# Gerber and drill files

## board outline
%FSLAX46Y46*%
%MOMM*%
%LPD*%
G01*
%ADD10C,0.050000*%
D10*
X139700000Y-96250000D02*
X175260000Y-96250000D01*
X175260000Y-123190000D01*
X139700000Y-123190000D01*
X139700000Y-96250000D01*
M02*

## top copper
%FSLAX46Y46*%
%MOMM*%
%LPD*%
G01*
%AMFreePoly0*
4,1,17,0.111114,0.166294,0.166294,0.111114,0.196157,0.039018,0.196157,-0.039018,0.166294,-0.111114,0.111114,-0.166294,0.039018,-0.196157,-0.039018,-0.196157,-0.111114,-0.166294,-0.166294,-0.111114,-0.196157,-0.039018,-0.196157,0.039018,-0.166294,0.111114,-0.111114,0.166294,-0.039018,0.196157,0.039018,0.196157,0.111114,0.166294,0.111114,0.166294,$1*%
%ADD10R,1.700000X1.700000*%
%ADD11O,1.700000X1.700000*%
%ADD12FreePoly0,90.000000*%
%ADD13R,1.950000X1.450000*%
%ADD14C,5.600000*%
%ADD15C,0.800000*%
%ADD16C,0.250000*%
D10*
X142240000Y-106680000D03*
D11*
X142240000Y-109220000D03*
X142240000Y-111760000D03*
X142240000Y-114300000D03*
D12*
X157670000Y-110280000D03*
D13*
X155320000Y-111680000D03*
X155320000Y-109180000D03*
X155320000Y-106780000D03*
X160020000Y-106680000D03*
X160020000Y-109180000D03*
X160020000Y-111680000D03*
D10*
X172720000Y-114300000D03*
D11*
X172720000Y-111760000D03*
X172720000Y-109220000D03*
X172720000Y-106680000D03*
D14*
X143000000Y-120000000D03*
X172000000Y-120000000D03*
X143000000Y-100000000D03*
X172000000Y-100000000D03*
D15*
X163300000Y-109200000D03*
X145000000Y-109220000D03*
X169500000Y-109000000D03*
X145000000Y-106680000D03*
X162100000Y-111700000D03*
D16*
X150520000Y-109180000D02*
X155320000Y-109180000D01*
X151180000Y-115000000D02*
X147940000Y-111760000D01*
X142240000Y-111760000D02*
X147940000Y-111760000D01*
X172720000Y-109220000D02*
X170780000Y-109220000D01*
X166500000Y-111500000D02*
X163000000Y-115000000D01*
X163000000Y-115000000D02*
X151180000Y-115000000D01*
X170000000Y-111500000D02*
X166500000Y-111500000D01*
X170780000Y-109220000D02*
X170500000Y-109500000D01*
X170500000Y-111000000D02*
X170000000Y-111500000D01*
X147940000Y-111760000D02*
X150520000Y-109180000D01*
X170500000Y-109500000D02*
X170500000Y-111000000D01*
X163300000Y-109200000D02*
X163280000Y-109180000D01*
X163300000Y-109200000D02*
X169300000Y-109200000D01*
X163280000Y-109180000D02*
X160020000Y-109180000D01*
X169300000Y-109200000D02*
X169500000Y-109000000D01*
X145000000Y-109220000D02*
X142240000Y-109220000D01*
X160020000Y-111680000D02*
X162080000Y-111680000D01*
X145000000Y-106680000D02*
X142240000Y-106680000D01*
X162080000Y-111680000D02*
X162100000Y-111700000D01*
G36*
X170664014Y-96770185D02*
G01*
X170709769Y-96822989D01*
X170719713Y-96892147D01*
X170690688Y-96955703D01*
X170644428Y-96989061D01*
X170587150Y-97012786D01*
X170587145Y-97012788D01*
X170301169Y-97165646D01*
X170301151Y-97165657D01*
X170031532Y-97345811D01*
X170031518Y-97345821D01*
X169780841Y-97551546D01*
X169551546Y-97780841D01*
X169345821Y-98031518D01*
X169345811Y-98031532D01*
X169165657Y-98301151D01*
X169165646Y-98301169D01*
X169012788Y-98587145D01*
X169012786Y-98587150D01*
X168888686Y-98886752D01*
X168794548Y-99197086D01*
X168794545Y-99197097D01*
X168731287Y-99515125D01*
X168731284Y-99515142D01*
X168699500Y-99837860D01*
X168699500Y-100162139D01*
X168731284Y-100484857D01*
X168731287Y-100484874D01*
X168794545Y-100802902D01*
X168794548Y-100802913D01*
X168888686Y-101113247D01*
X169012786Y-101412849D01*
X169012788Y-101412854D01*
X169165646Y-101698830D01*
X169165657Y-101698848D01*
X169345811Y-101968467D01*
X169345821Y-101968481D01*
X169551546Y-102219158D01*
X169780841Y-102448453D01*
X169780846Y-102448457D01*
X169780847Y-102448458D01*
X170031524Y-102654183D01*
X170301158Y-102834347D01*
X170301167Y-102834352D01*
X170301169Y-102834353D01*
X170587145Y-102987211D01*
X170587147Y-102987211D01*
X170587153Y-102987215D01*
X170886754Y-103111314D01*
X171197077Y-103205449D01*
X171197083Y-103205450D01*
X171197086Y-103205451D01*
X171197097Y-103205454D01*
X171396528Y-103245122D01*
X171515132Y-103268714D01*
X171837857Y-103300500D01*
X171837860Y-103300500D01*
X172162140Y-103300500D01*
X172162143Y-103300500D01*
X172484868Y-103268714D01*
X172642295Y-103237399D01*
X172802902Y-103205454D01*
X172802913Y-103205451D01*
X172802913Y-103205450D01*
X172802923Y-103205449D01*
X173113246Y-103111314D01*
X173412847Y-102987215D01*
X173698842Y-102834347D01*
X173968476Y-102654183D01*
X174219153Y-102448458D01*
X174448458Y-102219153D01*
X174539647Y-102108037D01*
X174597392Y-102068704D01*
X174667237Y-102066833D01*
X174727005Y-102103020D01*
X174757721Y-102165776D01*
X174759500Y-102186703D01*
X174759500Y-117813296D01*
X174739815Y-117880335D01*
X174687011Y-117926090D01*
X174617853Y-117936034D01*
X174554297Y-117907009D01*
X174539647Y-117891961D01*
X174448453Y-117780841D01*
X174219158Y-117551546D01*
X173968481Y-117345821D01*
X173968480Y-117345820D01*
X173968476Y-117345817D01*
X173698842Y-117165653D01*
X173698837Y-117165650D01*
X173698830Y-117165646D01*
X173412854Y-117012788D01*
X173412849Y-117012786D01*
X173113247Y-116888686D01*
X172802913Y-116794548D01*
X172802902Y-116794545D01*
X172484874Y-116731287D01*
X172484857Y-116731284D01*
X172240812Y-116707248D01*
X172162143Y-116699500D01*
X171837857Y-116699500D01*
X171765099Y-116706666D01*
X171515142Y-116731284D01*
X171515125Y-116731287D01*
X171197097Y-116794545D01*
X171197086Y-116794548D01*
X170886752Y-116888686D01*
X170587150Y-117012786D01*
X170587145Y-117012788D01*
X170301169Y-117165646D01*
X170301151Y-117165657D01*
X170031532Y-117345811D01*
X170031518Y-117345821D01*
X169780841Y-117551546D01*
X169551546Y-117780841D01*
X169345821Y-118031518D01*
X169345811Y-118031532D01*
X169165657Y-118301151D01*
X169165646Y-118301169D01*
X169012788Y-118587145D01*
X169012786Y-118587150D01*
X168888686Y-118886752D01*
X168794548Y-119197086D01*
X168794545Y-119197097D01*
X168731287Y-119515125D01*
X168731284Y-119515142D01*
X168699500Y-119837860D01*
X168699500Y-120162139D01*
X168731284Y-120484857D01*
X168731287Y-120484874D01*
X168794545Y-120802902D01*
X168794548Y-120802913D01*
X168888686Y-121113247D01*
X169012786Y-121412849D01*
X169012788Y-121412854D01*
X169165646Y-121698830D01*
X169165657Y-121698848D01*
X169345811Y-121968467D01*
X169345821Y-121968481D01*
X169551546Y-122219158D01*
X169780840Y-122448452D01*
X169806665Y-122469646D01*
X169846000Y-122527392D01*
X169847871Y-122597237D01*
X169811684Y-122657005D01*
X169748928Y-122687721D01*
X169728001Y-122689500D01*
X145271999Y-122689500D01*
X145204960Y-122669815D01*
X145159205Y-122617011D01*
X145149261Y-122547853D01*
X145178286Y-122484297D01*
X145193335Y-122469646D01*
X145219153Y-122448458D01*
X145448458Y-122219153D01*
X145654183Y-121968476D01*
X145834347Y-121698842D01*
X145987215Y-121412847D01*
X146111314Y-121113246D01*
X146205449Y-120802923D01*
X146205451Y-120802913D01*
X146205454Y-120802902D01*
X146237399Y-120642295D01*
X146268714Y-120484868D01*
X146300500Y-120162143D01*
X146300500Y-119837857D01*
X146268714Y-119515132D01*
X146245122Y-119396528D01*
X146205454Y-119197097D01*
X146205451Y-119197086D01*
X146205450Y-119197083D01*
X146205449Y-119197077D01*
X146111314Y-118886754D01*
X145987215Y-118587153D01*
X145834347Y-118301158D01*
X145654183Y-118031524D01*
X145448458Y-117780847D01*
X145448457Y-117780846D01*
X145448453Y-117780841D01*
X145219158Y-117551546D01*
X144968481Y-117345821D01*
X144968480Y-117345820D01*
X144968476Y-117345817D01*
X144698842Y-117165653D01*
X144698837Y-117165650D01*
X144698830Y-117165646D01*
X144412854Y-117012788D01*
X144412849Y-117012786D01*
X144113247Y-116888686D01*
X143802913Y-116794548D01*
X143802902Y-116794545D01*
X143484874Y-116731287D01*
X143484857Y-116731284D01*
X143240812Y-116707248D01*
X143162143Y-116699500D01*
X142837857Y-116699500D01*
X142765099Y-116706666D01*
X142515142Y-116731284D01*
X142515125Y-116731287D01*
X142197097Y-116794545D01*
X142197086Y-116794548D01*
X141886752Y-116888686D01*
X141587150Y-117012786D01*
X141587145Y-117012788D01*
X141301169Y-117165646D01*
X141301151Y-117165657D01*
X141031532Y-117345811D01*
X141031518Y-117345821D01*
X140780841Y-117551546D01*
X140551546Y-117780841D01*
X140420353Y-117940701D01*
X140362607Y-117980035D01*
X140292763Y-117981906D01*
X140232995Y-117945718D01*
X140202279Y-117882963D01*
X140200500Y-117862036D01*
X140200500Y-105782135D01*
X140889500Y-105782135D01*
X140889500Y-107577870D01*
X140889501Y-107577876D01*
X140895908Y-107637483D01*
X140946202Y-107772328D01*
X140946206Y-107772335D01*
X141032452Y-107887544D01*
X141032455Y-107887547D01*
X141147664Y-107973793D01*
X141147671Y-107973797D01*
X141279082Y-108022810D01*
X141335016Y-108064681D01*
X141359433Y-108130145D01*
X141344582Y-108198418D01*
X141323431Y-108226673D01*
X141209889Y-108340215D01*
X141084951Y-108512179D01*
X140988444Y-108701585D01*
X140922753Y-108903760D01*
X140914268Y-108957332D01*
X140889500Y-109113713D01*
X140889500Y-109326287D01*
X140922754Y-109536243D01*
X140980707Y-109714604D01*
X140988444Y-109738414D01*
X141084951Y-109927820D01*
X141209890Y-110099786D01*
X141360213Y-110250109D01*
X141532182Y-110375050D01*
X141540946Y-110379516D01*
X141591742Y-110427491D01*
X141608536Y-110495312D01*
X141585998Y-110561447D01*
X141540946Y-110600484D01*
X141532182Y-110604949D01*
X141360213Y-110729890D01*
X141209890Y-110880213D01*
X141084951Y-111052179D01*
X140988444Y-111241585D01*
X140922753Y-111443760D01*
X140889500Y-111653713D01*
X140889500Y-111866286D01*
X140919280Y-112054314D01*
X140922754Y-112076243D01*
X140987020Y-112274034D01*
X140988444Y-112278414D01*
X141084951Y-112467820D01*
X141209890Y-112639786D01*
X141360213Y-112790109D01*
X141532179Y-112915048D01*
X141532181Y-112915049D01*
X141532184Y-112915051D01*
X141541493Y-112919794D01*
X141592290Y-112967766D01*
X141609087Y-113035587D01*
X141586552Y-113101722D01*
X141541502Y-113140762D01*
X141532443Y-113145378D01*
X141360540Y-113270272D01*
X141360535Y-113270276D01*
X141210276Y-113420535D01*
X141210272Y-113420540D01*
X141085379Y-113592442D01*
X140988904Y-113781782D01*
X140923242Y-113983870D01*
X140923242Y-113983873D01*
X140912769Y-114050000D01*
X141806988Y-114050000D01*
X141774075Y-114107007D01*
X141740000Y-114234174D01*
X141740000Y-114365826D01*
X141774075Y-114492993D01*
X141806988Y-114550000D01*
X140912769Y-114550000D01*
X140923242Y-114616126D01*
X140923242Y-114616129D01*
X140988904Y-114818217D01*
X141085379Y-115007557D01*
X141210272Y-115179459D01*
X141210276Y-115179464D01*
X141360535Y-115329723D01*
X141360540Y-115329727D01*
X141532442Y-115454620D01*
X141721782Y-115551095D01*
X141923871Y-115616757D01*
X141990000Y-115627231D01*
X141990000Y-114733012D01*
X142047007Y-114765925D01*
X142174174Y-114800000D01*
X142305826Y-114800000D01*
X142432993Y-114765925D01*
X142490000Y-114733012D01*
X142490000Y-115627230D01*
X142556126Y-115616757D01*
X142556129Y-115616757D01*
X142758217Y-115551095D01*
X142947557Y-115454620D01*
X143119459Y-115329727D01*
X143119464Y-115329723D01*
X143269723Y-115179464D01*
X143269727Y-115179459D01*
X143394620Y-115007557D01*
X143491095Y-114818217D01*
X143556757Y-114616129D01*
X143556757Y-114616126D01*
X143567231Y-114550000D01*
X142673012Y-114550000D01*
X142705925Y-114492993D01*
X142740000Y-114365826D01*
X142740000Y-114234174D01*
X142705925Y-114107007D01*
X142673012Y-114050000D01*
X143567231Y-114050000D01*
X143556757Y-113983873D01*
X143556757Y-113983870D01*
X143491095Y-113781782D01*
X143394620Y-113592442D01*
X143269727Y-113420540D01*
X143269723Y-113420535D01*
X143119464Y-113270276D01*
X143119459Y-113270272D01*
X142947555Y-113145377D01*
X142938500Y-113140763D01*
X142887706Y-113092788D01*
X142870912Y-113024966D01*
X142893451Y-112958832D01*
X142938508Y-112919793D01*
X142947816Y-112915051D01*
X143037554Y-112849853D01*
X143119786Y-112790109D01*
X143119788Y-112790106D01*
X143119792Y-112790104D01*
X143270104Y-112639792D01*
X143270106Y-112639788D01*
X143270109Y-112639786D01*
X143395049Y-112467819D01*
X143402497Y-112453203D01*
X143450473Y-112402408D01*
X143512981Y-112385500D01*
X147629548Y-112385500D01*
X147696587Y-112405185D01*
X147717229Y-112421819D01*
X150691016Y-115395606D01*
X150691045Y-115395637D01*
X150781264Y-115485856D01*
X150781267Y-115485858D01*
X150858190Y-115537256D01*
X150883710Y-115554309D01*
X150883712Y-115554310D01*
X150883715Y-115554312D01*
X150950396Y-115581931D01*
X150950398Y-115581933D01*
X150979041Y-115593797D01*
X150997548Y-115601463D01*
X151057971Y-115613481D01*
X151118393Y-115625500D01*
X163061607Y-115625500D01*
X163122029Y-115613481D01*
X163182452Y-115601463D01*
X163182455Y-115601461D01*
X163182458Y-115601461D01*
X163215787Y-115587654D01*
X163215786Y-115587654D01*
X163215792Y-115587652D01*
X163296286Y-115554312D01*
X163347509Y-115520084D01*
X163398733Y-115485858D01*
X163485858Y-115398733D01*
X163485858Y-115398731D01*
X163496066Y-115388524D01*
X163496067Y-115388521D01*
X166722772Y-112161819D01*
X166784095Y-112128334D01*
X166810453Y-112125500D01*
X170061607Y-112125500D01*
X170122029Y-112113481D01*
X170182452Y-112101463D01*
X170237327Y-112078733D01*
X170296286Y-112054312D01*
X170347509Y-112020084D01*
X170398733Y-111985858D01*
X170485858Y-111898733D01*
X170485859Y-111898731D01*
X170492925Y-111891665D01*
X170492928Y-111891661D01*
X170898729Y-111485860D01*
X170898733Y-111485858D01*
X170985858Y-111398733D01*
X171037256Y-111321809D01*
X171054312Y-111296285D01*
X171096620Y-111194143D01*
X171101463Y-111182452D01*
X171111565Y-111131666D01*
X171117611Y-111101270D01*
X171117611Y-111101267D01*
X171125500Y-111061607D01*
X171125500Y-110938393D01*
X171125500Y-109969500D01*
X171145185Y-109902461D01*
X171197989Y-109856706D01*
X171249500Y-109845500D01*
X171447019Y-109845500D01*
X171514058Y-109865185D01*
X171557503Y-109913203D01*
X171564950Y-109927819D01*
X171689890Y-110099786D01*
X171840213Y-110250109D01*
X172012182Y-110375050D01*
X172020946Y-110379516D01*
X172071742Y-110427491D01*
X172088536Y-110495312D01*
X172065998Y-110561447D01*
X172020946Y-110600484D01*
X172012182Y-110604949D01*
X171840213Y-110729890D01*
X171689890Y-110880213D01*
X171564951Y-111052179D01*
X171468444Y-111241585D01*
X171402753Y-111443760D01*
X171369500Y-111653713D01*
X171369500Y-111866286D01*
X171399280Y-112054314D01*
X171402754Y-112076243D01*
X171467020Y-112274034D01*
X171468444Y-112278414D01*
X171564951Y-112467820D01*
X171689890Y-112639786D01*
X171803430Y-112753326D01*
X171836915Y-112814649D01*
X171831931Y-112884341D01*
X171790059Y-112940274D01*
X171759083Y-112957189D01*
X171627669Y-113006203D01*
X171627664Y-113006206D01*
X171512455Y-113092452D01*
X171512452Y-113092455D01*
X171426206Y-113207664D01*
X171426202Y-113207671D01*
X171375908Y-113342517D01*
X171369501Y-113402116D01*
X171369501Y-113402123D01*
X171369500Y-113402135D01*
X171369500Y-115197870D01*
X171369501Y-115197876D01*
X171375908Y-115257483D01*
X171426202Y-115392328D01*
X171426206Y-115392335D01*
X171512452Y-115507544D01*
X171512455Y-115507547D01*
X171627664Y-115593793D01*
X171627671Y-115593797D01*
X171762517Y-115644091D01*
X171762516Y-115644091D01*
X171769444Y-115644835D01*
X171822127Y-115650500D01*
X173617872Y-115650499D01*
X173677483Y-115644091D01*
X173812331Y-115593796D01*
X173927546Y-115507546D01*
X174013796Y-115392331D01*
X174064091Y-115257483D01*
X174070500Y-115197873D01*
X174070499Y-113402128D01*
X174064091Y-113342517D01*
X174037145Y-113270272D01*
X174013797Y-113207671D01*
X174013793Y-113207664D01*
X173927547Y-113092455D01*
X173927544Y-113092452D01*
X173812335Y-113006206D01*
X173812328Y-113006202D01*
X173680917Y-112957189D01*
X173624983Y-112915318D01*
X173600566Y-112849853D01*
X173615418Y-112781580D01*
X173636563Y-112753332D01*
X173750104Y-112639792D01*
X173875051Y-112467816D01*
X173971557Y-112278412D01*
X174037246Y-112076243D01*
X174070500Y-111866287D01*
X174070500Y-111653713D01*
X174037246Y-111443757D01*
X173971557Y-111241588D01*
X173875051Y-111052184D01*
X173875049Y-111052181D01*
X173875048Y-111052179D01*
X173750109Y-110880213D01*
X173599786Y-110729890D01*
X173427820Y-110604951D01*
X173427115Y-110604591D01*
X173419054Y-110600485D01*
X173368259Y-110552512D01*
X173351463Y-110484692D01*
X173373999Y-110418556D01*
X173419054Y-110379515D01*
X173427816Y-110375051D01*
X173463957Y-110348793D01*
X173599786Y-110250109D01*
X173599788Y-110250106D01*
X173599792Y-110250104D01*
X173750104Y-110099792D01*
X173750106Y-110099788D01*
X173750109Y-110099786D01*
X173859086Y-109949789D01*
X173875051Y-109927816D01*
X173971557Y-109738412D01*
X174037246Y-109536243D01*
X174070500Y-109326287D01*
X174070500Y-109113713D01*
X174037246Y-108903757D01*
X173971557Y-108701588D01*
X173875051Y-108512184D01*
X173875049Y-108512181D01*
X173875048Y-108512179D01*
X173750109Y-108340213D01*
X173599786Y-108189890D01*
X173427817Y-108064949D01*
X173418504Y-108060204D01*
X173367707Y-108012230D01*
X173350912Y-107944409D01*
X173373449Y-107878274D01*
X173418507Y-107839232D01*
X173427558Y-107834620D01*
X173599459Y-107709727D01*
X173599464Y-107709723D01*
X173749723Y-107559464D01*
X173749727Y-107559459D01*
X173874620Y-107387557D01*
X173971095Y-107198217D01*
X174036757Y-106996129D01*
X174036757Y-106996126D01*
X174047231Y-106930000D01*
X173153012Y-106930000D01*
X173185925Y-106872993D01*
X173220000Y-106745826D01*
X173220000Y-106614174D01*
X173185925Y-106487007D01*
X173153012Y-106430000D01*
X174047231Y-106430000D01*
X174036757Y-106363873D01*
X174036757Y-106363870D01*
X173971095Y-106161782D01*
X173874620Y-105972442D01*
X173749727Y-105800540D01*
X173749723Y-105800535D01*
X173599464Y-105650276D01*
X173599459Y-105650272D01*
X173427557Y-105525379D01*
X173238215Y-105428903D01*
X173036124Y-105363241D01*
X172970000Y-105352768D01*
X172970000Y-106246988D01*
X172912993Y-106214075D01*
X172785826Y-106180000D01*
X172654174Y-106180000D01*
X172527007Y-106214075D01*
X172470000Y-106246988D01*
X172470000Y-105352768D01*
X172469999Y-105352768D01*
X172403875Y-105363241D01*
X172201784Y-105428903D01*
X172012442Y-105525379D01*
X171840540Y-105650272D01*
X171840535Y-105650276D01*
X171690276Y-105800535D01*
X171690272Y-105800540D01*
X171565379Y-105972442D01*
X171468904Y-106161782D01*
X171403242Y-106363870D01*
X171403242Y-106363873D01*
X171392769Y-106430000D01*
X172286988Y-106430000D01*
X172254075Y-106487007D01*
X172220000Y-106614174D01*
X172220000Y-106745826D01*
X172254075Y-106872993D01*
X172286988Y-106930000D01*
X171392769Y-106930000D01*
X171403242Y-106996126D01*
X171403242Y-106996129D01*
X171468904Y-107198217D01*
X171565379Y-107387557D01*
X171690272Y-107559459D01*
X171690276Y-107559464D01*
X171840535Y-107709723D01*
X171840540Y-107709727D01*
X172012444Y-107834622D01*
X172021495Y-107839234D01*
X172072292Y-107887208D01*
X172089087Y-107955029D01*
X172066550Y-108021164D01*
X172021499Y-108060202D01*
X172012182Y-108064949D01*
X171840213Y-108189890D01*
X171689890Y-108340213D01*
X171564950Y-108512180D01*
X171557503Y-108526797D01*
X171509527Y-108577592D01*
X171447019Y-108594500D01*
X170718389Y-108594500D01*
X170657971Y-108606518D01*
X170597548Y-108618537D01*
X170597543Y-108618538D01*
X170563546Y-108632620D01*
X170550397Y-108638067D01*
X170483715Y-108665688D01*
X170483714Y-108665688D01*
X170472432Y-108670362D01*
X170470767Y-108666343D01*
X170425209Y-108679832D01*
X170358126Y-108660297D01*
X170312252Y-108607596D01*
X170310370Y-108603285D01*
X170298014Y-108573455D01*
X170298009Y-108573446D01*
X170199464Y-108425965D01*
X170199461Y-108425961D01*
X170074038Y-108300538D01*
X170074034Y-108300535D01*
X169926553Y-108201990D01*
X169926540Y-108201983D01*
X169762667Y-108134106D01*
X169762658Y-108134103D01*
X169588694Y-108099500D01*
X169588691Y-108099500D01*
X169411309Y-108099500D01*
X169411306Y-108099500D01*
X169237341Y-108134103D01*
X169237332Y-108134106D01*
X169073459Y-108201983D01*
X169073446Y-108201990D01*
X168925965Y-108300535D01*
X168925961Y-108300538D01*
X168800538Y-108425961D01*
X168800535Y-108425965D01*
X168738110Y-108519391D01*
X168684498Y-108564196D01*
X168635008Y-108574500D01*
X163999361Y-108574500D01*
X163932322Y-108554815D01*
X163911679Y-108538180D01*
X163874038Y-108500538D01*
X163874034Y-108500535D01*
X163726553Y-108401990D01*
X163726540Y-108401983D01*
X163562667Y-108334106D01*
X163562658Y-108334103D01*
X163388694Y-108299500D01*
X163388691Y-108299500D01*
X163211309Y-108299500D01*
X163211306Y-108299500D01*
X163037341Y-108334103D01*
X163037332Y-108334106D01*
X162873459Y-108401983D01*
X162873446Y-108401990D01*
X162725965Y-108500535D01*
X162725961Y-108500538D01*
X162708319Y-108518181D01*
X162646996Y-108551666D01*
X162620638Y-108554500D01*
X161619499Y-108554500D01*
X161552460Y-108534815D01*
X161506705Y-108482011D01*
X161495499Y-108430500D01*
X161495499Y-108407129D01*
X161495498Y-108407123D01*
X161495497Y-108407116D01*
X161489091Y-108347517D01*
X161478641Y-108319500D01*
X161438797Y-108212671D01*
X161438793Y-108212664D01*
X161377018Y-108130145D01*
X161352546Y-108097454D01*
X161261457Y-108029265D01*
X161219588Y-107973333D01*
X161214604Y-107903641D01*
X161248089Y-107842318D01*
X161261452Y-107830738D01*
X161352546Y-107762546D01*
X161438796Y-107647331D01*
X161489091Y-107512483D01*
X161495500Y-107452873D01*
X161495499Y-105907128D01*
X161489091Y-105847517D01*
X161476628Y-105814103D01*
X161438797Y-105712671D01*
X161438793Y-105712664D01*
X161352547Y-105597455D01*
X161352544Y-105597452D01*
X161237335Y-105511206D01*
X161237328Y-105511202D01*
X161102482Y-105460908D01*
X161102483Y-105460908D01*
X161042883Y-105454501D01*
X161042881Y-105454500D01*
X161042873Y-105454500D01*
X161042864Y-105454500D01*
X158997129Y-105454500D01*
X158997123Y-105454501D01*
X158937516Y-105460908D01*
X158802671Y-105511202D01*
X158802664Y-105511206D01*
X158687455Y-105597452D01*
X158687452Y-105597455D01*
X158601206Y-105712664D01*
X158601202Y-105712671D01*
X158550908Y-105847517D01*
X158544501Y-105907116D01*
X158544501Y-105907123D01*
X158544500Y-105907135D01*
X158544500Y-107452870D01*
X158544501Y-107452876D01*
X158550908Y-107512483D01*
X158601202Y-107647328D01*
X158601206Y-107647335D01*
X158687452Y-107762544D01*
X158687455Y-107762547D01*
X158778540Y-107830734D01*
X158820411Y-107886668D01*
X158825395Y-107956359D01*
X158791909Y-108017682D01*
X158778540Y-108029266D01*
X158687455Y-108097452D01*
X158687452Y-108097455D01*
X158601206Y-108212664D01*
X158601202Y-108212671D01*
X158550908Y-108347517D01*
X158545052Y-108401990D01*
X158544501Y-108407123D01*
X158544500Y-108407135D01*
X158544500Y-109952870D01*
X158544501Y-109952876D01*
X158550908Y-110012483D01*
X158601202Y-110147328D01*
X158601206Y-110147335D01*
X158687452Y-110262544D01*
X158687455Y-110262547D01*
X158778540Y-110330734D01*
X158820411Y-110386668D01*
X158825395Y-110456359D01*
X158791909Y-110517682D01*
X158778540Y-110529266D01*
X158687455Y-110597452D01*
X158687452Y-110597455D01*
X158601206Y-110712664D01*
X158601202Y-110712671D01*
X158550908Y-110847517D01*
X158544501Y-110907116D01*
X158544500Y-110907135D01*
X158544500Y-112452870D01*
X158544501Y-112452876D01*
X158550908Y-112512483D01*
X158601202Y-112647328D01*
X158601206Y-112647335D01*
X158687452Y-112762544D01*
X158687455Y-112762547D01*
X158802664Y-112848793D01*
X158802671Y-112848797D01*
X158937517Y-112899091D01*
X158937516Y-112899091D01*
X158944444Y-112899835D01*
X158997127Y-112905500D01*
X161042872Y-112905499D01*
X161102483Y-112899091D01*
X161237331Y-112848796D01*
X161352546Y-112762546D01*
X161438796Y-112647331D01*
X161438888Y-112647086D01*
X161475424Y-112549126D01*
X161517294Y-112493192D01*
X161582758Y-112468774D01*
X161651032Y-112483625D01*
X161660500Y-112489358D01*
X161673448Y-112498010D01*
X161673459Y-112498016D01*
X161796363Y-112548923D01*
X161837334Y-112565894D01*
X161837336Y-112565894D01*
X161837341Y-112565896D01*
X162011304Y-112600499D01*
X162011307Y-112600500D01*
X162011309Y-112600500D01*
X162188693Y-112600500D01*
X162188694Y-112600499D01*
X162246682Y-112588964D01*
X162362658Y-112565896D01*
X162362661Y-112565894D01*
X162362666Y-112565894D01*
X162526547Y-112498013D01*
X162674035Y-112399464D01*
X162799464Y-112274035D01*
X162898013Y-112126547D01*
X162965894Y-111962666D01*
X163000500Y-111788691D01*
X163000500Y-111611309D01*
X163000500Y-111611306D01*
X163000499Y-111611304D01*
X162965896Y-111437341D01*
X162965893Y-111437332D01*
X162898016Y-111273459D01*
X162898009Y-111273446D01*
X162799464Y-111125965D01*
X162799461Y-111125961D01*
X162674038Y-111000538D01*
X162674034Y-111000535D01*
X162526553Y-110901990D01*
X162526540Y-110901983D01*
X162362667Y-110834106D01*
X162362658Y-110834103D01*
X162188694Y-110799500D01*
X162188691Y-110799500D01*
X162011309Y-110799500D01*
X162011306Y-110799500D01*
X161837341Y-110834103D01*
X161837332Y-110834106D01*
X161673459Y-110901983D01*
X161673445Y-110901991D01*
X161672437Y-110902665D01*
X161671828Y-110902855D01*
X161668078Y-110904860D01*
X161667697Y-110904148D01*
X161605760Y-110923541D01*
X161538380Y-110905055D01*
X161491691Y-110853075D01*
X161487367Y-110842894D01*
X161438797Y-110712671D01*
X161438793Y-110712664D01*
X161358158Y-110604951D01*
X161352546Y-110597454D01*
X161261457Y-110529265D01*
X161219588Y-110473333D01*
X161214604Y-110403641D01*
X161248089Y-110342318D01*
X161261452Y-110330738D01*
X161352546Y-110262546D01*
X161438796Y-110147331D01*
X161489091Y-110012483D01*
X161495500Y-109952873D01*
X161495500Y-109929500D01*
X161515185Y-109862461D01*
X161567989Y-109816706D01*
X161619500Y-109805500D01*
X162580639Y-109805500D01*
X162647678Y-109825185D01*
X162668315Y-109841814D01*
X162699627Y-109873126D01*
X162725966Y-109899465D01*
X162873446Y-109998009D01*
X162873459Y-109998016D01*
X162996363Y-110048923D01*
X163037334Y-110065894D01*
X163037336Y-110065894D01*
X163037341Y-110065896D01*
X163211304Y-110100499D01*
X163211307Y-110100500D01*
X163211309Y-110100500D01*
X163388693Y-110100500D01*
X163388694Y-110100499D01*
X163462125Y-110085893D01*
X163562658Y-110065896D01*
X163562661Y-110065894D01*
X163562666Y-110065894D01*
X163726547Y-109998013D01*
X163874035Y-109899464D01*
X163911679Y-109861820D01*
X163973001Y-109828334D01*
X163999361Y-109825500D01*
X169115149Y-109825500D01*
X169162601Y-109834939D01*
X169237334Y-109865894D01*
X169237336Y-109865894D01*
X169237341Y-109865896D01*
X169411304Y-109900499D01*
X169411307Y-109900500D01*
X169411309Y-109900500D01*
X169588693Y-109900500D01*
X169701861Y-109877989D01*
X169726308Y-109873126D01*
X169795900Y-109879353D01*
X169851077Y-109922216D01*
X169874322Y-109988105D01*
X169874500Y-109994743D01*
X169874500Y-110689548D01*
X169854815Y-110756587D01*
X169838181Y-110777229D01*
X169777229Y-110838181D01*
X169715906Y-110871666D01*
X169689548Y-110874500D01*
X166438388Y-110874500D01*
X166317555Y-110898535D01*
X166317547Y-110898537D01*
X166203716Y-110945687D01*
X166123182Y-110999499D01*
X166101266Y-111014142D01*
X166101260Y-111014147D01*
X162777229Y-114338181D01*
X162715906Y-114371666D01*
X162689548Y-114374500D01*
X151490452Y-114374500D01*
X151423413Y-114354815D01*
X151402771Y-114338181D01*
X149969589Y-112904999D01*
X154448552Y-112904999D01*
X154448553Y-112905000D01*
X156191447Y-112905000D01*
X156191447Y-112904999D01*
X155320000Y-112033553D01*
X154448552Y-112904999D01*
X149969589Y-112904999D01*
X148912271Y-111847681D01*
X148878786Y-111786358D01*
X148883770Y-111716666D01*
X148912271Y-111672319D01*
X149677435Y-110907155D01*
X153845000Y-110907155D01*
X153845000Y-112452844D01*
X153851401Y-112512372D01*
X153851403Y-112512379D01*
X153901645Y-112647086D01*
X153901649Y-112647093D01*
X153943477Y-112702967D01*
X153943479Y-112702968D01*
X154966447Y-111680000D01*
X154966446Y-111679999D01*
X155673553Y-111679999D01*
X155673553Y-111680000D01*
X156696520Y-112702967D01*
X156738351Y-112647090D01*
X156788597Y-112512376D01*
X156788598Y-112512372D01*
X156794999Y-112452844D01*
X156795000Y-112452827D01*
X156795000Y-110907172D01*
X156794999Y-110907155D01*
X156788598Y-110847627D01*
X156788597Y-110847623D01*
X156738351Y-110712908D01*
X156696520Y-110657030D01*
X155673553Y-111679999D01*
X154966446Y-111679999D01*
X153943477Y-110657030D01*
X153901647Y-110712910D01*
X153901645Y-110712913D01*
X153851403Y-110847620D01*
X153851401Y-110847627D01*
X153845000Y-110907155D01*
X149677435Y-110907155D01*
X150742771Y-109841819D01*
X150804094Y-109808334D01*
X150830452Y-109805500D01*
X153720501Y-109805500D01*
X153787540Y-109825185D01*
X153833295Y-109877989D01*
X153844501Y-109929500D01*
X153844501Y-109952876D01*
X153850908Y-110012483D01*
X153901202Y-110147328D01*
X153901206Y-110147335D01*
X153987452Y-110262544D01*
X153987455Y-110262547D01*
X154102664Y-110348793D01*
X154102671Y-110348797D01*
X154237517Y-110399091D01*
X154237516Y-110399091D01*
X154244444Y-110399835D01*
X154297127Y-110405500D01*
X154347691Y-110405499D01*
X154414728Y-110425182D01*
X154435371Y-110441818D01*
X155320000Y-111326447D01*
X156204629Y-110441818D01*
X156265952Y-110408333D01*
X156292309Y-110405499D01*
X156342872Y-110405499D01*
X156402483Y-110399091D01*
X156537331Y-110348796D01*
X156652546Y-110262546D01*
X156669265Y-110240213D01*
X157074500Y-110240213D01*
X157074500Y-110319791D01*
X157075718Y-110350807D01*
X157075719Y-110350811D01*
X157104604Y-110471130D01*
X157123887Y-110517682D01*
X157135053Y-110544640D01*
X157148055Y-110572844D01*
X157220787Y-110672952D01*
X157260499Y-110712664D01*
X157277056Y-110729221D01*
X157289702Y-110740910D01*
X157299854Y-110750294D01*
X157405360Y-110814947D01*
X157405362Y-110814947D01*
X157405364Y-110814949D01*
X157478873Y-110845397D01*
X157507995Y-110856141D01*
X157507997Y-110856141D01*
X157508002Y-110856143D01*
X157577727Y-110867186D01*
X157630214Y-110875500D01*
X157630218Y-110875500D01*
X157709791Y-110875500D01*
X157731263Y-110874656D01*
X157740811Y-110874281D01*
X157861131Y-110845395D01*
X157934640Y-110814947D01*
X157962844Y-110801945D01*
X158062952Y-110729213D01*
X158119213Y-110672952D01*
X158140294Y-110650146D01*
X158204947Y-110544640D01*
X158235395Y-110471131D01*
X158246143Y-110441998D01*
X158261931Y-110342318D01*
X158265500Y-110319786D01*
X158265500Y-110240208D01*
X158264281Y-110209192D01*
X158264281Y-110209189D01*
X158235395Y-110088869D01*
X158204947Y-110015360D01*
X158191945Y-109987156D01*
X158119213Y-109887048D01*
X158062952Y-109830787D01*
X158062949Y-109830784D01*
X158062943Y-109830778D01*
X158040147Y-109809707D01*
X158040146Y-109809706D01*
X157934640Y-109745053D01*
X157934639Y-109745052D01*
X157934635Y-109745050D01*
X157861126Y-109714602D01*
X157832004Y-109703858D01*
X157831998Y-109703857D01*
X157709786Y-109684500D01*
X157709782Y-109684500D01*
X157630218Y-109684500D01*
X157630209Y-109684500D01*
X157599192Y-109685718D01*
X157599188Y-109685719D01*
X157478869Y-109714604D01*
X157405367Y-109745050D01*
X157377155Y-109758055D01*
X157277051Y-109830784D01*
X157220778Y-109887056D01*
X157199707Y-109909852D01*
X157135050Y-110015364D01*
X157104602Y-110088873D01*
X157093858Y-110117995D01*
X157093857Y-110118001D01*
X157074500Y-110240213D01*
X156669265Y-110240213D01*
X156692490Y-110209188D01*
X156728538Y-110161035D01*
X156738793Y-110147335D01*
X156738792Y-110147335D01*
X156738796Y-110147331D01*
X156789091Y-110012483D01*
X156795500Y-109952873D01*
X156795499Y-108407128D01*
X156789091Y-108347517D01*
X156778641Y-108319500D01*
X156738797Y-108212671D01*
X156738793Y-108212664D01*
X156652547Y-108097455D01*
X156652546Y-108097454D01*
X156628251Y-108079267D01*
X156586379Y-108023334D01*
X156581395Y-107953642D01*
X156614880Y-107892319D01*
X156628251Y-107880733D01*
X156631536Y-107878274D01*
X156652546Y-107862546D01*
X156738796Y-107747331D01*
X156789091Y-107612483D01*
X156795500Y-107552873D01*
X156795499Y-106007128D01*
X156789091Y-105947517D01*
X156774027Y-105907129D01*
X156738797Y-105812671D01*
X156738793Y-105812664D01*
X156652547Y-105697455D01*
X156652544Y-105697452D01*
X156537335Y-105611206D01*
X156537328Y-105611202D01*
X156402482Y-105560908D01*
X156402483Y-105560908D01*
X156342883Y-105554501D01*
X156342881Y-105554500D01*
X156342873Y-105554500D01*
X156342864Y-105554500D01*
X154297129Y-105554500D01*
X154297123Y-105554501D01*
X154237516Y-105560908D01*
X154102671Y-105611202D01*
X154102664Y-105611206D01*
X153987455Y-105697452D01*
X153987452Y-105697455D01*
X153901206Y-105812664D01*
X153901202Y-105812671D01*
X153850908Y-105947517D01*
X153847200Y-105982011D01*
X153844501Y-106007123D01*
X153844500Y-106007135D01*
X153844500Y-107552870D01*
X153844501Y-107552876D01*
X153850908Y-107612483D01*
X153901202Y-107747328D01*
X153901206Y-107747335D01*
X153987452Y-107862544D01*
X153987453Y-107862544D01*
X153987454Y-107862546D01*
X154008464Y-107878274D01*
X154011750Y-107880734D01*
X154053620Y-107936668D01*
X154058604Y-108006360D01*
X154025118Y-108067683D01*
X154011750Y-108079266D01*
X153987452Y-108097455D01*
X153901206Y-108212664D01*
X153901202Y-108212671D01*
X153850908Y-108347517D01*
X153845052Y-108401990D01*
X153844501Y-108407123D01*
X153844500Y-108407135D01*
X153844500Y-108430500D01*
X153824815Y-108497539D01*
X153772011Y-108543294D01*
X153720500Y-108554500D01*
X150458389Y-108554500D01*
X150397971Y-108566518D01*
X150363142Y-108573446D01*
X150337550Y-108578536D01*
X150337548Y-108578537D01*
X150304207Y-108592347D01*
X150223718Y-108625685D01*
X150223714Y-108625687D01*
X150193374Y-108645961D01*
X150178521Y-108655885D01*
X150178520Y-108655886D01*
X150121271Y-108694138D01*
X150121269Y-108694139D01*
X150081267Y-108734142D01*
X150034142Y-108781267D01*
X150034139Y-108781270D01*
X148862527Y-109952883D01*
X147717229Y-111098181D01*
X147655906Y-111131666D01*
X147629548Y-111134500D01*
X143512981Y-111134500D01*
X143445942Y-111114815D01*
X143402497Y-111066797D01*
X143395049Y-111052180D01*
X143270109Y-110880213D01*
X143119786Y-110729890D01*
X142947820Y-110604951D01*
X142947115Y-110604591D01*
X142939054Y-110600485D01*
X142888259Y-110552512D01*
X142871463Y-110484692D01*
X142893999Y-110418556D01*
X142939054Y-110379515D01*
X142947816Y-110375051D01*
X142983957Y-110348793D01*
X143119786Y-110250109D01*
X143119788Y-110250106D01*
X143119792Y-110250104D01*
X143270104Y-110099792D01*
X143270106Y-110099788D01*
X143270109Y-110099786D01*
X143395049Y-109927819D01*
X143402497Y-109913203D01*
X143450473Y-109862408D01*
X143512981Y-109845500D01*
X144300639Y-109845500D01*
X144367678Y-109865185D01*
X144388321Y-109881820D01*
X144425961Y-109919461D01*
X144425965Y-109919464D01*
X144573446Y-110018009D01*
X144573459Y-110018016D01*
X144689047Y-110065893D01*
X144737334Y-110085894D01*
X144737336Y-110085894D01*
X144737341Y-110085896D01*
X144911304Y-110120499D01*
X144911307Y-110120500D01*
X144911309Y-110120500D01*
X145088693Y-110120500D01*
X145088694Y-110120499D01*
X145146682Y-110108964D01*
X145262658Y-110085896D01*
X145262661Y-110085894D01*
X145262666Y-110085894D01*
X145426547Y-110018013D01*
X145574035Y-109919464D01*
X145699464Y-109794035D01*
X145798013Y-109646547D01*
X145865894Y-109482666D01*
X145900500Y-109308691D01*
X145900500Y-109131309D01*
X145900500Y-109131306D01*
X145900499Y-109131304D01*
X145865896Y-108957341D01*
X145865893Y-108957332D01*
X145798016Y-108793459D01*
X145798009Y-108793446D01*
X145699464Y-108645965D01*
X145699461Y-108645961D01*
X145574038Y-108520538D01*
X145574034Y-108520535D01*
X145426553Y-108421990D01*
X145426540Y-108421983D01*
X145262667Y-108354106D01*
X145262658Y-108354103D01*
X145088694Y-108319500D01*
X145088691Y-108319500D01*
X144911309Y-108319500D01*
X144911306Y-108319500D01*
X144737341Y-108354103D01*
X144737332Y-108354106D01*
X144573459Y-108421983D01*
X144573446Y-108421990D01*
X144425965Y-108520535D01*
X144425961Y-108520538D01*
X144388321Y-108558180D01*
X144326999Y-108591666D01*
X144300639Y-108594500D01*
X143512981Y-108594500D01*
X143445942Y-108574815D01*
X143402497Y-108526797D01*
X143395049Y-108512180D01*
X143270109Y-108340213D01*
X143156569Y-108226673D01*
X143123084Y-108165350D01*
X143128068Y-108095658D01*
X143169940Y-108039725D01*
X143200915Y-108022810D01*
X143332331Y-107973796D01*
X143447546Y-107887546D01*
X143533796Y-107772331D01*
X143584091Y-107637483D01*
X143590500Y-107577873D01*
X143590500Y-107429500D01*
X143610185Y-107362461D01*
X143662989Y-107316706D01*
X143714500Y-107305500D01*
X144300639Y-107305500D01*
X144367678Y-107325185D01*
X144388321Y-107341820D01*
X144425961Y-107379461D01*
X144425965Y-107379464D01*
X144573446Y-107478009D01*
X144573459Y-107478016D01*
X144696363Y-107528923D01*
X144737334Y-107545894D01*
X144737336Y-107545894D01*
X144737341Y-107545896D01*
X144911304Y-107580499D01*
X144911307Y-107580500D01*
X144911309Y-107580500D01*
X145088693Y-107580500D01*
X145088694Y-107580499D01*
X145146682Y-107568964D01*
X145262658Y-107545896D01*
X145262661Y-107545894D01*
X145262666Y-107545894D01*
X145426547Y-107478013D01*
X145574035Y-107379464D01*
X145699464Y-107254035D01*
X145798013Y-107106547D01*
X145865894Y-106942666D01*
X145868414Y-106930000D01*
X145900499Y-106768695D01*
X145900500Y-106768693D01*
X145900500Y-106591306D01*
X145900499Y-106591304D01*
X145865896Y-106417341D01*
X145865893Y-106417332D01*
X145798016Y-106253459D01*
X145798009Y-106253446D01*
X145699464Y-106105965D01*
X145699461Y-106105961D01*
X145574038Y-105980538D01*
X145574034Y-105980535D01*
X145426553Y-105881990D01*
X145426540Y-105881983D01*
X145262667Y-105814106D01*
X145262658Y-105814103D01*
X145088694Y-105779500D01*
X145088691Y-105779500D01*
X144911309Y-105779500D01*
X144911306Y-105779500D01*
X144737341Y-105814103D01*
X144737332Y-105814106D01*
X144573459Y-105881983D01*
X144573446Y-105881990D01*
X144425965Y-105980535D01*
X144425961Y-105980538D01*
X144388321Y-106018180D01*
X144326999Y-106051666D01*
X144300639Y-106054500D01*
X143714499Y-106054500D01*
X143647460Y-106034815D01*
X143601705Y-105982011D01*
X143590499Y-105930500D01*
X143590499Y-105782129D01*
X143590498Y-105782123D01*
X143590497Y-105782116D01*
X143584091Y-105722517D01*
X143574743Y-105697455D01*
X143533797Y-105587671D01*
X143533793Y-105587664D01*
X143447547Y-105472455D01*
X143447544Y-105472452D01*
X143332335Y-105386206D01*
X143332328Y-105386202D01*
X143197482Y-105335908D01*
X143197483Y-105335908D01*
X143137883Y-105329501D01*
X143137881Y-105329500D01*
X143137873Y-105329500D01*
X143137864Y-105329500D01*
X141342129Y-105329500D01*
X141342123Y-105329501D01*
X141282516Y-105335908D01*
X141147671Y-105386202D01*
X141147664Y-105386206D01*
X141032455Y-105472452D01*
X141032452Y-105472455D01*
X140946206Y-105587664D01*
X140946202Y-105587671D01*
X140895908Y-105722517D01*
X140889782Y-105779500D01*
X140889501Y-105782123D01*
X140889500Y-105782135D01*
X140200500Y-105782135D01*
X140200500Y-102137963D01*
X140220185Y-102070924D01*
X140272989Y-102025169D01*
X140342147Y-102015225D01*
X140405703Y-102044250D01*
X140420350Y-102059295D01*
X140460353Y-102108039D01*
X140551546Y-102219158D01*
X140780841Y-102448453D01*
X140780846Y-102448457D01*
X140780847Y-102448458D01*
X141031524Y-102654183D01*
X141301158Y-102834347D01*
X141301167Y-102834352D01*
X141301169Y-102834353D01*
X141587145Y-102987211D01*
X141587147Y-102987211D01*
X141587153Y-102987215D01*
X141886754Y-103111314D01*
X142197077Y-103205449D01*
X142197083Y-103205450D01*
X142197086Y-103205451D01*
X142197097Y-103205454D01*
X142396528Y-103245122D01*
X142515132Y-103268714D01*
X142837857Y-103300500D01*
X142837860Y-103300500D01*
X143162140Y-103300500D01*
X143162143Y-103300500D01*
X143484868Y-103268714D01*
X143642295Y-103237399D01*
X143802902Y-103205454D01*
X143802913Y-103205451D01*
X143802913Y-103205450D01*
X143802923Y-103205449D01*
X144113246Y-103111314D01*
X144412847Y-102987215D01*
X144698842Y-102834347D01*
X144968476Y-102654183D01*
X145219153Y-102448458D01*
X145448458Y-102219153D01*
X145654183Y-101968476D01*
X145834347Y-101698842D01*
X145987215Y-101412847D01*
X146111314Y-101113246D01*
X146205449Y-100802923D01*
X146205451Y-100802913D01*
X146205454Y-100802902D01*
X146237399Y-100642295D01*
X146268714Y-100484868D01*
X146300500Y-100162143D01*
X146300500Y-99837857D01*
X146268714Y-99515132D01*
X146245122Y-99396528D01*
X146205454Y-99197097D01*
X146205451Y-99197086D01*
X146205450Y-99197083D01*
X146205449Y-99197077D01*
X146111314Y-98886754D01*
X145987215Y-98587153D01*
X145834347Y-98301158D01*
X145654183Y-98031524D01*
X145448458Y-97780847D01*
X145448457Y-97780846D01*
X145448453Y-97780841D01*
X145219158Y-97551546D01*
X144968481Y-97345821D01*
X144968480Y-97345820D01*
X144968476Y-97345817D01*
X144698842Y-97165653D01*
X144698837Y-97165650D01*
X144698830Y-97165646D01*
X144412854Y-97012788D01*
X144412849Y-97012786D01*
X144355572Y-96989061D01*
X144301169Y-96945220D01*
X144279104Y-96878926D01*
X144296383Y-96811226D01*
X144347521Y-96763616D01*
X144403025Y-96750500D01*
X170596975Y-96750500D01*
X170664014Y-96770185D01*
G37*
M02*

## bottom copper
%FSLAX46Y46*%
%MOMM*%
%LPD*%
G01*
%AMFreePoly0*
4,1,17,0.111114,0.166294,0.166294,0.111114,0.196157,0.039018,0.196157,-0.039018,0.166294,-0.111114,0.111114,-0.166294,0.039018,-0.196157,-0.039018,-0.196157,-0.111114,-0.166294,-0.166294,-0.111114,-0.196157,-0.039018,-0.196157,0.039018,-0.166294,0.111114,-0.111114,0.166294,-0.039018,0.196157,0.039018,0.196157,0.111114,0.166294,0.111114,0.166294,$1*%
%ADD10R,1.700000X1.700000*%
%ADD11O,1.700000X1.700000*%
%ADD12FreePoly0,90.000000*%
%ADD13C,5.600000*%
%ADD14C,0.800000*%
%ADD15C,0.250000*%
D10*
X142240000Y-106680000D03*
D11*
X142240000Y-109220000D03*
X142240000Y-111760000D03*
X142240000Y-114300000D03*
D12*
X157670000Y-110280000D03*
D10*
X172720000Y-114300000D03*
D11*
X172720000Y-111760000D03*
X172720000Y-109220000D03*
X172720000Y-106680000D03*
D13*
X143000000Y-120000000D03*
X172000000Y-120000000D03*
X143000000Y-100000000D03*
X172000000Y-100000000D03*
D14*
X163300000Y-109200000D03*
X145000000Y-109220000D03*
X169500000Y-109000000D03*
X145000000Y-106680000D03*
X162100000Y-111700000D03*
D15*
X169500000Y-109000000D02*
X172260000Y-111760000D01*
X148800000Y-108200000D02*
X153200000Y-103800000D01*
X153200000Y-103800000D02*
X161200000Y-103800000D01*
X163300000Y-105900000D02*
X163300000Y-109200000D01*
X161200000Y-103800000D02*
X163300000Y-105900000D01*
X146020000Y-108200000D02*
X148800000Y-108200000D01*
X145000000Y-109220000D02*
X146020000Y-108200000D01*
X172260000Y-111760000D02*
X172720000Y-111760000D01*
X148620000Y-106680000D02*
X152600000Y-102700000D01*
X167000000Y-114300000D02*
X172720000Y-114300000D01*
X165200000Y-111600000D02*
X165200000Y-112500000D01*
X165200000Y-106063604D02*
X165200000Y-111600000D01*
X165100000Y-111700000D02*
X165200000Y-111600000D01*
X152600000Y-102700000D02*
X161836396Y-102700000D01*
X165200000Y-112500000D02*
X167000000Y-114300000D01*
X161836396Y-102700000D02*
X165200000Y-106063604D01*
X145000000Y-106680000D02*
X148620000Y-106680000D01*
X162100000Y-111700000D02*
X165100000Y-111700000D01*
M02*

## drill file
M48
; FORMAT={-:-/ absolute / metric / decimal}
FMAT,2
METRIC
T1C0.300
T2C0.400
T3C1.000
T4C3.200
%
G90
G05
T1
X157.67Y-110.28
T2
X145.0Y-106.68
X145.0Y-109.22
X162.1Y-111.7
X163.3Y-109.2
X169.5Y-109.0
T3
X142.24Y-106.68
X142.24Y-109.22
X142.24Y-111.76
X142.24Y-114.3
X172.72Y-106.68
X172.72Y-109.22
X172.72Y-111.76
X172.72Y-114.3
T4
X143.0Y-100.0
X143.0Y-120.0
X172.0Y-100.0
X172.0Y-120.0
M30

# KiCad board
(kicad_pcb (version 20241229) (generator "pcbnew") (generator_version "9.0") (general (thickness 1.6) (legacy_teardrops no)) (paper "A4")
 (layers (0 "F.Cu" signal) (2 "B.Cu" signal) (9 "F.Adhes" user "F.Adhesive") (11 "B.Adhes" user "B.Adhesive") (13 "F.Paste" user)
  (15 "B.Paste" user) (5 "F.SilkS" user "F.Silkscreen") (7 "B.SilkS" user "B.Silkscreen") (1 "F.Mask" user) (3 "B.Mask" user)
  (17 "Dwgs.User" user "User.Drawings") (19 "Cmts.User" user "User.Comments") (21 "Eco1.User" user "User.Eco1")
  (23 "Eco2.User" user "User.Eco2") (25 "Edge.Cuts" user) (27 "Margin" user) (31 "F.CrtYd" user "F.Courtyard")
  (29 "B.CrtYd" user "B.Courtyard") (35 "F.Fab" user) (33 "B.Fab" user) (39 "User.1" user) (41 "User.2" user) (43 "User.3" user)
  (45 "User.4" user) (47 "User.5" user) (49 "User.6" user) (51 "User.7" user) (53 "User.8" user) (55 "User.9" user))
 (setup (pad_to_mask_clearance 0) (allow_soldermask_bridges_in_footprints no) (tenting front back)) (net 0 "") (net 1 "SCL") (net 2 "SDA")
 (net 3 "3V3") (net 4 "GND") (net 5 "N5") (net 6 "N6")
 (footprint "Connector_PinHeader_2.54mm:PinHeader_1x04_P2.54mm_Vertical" (layer "F.Cu") (at 142.24 106.68)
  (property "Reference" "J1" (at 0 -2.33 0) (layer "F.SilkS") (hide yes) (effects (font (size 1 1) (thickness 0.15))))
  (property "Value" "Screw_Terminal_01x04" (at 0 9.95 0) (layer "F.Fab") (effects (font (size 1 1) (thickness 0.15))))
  (pad "1" thru_hole rect (at 0 0) (size 1.7 1.7) (drill 1) (layers "*.Cu" "*.Mask") (remove_unused_layers no) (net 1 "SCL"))
  (pad "2" thru_hole oval (at 0 2.54) (size 1.7 1.7) (drill 1) (layers "*.Cu" "*.Mask") (remove_unused_layers no) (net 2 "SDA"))
  (pad "3" thru_hole oval (at 0 5.08) (size 1.7 1.7) (drill 1) (layers "*.Cu" "*.Mask") (remove_unused_layers no) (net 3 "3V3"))
  (pad "4" thru_hole oval (at 0 7.62) (size 1.7 1.7) (drill 1) (layers "*.Cu" "*.Mask") (remove_unused_layers no) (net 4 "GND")))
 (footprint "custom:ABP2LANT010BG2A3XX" (layer "F.Cu") (at 154.07 113.28 90)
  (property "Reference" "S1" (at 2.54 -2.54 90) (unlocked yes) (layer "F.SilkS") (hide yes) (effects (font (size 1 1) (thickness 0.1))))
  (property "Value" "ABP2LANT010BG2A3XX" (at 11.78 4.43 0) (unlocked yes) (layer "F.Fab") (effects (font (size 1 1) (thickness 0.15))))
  (pad "" thru_hole custom (at 3 3.6 90) (size 0.4 0.4) (drill 0.3) (layers "*.Cu" "*.Mask") (remove_unused_layers no)
   (solder_mask_margin 0.6) (clearance 0.39) (thermal_bridge_angle 90) (options (clearance outline) (anchor circle)) (primitives))
  (pad "1" smd rect (at 1.6 1.25 90) (size 1.45 1.95) (layers "F.Cu" "F.Mask" "F.Paste") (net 4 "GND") (thermal_bridge_angle 45))
  (pad "2" smd rect (at 4.1 1.25 90) (size 1.45 1.95) (layers "F.Cu" "F.Mask" "F.Paste") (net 3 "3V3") (thermal_bridge_angle 45))
  (pad "3" smd rect (at 6.5 1.25 90) (size 1.45 1.95) (layers "F.Cu" "F.Mask" "F.Paste") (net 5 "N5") (thermal_bridge_angle 45))
  (pad "4" smd rect (at 6.6 5.95 90) (size 1.45 1.95) (layers "F.Cu" "F.Mask" "F.Paste") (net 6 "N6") (thermal_bridge_angle 45))
  (pad "5" smd rect (at 4.1 5.95 90) (size 1.45 1.95) (layers "F.Cu" "F.Mask" "F.Paste") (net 2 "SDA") (thermal_bridge_angle 45))
  (pad "6" smd rect (at 1.6 5.95 90) (size 1.45 1.95) (layers "F.Cu" "F.Mask" "F.Paste") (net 1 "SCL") (thermal_bridge_angle 45)))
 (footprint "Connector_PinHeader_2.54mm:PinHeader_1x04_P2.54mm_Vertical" (layer "F.Cu") (at 172.72 114.3 180)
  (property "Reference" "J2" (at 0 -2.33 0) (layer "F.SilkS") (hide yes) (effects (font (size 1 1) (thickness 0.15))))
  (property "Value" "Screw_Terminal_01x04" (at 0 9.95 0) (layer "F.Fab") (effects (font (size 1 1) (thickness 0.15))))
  (pad "1" thru_hole rect (at 0 0 180) (size 1.7 1.7) (drill 1) (layers "*.Cu" "*.Mask") (remove_unused_layers no) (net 1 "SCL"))
  (pad "2" thru_hole oval (at 0 2.54 180) (size 1.7 1.7) (drill 1) (layers "*.Cu" "*.Mask") (remove_unused_layers no) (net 2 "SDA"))
  (pad "3" thru_hole oval (at 0 5.08 180) (size 1.7 1.7) (drill 1) (layers "*.Cu" "*.Mask") (remove_unused_layers no) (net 3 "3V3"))
  (pad "4" thru_hole oval (at 0 7.62 180) (size 1.7 1.7) (drill 1) (layers "*.Cu" "*.Mask") (remove_unused_layers no) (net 4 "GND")))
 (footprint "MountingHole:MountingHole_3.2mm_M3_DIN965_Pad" (layer "F.Cu") (at 143 120)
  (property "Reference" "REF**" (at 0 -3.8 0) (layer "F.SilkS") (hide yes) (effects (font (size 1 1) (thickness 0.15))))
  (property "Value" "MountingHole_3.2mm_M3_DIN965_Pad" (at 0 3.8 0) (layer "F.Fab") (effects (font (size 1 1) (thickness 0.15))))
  (pad "1" thru_hole circle (at 0 0) (size 5.6 5.6) (drill 3.2) (layers "*.Cu" "*.Mask") (remove_unused_layers no)))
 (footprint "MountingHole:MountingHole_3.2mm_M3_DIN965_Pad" (layer "F.Cu") (at 172 120)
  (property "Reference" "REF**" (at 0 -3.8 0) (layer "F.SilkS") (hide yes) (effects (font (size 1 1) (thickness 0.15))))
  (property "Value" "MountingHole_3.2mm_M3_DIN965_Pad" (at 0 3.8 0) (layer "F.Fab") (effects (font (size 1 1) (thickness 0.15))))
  (pad "1" thru_hole circle (at 0 0) (size 5.6 5.6) (drill 3.2) (layers "*.Cu" "*.Mask") (remove_unused_layers no)))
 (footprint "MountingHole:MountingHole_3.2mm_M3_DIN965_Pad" (layer "F.Cu") (at 143 100)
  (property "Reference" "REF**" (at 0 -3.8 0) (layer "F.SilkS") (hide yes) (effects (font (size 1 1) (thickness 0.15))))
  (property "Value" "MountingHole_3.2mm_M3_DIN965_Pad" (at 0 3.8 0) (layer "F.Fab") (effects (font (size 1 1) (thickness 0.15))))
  (pad "1" thru_hole circle (at 0 0) (size 5.6 5.6) (drill 3.2) (layers "*.Cu" "*.Mask") (remove_unused_layers no)))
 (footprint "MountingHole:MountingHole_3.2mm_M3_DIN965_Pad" (layer "F.Cu") (at 172 100)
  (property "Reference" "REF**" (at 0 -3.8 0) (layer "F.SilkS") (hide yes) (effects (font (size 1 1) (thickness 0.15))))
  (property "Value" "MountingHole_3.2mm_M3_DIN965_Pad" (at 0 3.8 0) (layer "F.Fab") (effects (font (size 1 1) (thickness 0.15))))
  (pad "1" thru_hole circle (at 0 0) (size 5.6 5.6) (drill 3.2) (layers "*.Cu" "*.Mask") (remove_unused_layers no)))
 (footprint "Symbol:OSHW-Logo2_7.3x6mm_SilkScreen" (layer "F.Cu") (at 158 119.5)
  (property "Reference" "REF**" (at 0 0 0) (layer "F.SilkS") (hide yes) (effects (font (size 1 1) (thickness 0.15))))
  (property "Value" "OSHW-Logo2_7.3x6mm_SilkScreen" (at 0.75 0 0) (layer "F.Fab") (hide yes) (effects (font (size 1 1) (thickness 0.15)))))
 (gr_rect (start 139.7 96.25) (end 175.26 123.19) (stroke (width 0.05) (type default)) (fill no) (layer "Edge.Cuts"))
 (segment (start 150.52 109.18) (end 155.32 109.18) (width 0.25) (layer "F.Cu") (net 3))
 (segment (start 151.18 115) (end 147.94 111.76) (width 0.25) (layer "F.Cu") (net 3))
 (segment (start 142.24 111.76) (end 147.94 111.76) (width 0.25) (layer "F.Cu") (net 3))
 (segment (start 172.72 109.22) (end 170.78 109.22) (width 0.25) (layer "F.Cu") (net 3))
 (segment (start 166.5 111.5) (end 163 115) (width 0.25) (layer "F.Cu") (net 3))
 (segment (start 163 115) (end 151.18 115) (width 0.25) (layer "F.Cu") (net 3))
 (segment (start 170 111.5) (end 166.5 111.5) (width 0.25) (layer "F.Cu") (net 3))
 (segment (start 170.78 109.22) (end 170.5 109.5) (width 0.25) (layer "F.Cu") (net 3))
 (segment (start 170.5 111) (end 170 111.5) (width 0.25) (layer "F.Cu") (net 3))
 (segment (start 147.94 111.76) (end 150.52 109.18) (width 0.25) (layer "F.Cu") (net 3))
 (segment (start 170.5 109.5) (end 170.5 111) (width 0.25) (layer "F.Cu") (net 3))
 (segment (start 163.3 109.2) (end 163.28 109.18) (width 0.25) (layer "F.Cu") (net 2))
 (segment (start 163.3 109.2) (end 169.3 109.2) (width 0.25) (layer "F.Cu") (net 2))
 (segment (start 163.28 109.18) (end 160.02 109.18) (width 0.25) (layer "F.Cu") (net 2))
 (segment (start 169.3 109.2) (end 169.5 109) (width 0.25) (layer "F.Cu") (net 2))
 (segment (start 145 109.22) (end 142.24 109.22) (width 0.25) (layer "F.Cu") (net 2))
 (via (at 163.3 109.2) (size 0.8) (drill 0.4) (layers "F.Cu" "B.Cu") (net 2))
 (via (at 145 109.22) (size 0.8) (drill 0.4) (layers "F.Cu" "B.Cu") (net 2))
 (via (at 169.5 109) (size 0.8) (drill 0.4) (layers "F.Cu" "B.Cu") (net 2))
 (segment (start 169.5 109) (end 172.26 111.76) (width 0.25) (layer "B.Cu") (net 2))
 (segment (start 148.8 108.2) (end 153.2 103.8) (width 0.25) (layer "B.Cu") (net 2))
 (segment (start 153.2 103.8) (end 161.2 103.8) (width 0.25) (layer "B.Cu") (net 2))
 (segment (start 163.3 105.9) (end 163.3 109.2) (width 0.25) (layer "B.Cu") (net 2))
 (segment (start 161.2 103.8) (end 163.3 105.9) (width 0.25) (layer "B.Cu") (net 2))
 (segment (start 146.02 108.2) (end 148.8 108.2) (width 0.25) (layer "B.Cu") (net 2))
 (segment (start 145 109.22) (end 146.02 108.2) (width 0.25) (layer "B.Cu") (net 2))
 (segment (start 172.26 111.76) (end 172.72 111.76) (width 0.25) (layer "B.Cu") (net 2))
 (segment (start 160.02 111.68) (end 162.08 111.68) (width 0.25) (layer "F.Cu") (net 1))
 (segment (start 145 106.68) (end 142.24 106.68) (width 0.25) (layer "F.Cu") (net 1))
 (segment (start 162.08 111.68) (end 162.1 111.7) (width 0.25) (layer "F.Cu") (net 1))
 (via (at 145 106.68) (size 0.8) (drill 0.4) (layers "F.Cu" "B.Cu") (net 1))
 (via (at 162.1 111.7) (size 0.8) (drill 0.4) (layers "F.Cu" "B.Cu") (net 1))
 (segment (start 148.62 106.68) (end 152.6 102.7) (width 0.25) (layer "B.Cu") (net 1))
 (segment (start 167 114.3) (end 172.72 114.3) (width 0.25) (layer "B.Cu") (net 1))
 (segment (start 165.2 111.6) (end 165.2 112.5) (width 0.25) (layer "B.Cu") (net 1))
 (segment (start 165.2 106.063604) (end 165.2 111.6) (width 0.25) (layer "B.Cu") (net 1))
 (segment (start 165.1 111.7) (end 165.2 111.6) (width 0.25) (layer "B.Cu") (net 1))
 (segment (start 152.6 102.7) (end 161.836396 102.7) (width 0.25) (layer "B.Cu") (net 1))
 (segment (start 165.2 112.5) (end 167 114.3) (width 0.25) (layer "B.Cu") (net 1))
 (segment (start 161.836396 102.7) (end 165.2 106.063604) (width 0.25) (layer "B.Cu") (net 1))
 (segment (start 145 106.68) (end 148.62 106.68) (width 0.25) (layer "B.Cu") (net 1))
 (segment (start 162.1 111.7) (end 165.1 111.7) (width 0.25) (layer "B.Cu") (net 1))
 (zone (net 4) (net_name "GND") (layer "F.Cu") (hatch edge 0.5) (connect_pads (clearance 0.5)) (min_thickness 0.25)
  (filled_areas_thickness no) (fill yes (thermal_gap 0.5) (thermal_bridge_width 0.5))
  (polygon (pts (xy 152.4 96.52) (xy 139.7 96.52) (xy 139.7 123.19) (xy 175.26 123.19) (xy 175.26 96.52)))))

